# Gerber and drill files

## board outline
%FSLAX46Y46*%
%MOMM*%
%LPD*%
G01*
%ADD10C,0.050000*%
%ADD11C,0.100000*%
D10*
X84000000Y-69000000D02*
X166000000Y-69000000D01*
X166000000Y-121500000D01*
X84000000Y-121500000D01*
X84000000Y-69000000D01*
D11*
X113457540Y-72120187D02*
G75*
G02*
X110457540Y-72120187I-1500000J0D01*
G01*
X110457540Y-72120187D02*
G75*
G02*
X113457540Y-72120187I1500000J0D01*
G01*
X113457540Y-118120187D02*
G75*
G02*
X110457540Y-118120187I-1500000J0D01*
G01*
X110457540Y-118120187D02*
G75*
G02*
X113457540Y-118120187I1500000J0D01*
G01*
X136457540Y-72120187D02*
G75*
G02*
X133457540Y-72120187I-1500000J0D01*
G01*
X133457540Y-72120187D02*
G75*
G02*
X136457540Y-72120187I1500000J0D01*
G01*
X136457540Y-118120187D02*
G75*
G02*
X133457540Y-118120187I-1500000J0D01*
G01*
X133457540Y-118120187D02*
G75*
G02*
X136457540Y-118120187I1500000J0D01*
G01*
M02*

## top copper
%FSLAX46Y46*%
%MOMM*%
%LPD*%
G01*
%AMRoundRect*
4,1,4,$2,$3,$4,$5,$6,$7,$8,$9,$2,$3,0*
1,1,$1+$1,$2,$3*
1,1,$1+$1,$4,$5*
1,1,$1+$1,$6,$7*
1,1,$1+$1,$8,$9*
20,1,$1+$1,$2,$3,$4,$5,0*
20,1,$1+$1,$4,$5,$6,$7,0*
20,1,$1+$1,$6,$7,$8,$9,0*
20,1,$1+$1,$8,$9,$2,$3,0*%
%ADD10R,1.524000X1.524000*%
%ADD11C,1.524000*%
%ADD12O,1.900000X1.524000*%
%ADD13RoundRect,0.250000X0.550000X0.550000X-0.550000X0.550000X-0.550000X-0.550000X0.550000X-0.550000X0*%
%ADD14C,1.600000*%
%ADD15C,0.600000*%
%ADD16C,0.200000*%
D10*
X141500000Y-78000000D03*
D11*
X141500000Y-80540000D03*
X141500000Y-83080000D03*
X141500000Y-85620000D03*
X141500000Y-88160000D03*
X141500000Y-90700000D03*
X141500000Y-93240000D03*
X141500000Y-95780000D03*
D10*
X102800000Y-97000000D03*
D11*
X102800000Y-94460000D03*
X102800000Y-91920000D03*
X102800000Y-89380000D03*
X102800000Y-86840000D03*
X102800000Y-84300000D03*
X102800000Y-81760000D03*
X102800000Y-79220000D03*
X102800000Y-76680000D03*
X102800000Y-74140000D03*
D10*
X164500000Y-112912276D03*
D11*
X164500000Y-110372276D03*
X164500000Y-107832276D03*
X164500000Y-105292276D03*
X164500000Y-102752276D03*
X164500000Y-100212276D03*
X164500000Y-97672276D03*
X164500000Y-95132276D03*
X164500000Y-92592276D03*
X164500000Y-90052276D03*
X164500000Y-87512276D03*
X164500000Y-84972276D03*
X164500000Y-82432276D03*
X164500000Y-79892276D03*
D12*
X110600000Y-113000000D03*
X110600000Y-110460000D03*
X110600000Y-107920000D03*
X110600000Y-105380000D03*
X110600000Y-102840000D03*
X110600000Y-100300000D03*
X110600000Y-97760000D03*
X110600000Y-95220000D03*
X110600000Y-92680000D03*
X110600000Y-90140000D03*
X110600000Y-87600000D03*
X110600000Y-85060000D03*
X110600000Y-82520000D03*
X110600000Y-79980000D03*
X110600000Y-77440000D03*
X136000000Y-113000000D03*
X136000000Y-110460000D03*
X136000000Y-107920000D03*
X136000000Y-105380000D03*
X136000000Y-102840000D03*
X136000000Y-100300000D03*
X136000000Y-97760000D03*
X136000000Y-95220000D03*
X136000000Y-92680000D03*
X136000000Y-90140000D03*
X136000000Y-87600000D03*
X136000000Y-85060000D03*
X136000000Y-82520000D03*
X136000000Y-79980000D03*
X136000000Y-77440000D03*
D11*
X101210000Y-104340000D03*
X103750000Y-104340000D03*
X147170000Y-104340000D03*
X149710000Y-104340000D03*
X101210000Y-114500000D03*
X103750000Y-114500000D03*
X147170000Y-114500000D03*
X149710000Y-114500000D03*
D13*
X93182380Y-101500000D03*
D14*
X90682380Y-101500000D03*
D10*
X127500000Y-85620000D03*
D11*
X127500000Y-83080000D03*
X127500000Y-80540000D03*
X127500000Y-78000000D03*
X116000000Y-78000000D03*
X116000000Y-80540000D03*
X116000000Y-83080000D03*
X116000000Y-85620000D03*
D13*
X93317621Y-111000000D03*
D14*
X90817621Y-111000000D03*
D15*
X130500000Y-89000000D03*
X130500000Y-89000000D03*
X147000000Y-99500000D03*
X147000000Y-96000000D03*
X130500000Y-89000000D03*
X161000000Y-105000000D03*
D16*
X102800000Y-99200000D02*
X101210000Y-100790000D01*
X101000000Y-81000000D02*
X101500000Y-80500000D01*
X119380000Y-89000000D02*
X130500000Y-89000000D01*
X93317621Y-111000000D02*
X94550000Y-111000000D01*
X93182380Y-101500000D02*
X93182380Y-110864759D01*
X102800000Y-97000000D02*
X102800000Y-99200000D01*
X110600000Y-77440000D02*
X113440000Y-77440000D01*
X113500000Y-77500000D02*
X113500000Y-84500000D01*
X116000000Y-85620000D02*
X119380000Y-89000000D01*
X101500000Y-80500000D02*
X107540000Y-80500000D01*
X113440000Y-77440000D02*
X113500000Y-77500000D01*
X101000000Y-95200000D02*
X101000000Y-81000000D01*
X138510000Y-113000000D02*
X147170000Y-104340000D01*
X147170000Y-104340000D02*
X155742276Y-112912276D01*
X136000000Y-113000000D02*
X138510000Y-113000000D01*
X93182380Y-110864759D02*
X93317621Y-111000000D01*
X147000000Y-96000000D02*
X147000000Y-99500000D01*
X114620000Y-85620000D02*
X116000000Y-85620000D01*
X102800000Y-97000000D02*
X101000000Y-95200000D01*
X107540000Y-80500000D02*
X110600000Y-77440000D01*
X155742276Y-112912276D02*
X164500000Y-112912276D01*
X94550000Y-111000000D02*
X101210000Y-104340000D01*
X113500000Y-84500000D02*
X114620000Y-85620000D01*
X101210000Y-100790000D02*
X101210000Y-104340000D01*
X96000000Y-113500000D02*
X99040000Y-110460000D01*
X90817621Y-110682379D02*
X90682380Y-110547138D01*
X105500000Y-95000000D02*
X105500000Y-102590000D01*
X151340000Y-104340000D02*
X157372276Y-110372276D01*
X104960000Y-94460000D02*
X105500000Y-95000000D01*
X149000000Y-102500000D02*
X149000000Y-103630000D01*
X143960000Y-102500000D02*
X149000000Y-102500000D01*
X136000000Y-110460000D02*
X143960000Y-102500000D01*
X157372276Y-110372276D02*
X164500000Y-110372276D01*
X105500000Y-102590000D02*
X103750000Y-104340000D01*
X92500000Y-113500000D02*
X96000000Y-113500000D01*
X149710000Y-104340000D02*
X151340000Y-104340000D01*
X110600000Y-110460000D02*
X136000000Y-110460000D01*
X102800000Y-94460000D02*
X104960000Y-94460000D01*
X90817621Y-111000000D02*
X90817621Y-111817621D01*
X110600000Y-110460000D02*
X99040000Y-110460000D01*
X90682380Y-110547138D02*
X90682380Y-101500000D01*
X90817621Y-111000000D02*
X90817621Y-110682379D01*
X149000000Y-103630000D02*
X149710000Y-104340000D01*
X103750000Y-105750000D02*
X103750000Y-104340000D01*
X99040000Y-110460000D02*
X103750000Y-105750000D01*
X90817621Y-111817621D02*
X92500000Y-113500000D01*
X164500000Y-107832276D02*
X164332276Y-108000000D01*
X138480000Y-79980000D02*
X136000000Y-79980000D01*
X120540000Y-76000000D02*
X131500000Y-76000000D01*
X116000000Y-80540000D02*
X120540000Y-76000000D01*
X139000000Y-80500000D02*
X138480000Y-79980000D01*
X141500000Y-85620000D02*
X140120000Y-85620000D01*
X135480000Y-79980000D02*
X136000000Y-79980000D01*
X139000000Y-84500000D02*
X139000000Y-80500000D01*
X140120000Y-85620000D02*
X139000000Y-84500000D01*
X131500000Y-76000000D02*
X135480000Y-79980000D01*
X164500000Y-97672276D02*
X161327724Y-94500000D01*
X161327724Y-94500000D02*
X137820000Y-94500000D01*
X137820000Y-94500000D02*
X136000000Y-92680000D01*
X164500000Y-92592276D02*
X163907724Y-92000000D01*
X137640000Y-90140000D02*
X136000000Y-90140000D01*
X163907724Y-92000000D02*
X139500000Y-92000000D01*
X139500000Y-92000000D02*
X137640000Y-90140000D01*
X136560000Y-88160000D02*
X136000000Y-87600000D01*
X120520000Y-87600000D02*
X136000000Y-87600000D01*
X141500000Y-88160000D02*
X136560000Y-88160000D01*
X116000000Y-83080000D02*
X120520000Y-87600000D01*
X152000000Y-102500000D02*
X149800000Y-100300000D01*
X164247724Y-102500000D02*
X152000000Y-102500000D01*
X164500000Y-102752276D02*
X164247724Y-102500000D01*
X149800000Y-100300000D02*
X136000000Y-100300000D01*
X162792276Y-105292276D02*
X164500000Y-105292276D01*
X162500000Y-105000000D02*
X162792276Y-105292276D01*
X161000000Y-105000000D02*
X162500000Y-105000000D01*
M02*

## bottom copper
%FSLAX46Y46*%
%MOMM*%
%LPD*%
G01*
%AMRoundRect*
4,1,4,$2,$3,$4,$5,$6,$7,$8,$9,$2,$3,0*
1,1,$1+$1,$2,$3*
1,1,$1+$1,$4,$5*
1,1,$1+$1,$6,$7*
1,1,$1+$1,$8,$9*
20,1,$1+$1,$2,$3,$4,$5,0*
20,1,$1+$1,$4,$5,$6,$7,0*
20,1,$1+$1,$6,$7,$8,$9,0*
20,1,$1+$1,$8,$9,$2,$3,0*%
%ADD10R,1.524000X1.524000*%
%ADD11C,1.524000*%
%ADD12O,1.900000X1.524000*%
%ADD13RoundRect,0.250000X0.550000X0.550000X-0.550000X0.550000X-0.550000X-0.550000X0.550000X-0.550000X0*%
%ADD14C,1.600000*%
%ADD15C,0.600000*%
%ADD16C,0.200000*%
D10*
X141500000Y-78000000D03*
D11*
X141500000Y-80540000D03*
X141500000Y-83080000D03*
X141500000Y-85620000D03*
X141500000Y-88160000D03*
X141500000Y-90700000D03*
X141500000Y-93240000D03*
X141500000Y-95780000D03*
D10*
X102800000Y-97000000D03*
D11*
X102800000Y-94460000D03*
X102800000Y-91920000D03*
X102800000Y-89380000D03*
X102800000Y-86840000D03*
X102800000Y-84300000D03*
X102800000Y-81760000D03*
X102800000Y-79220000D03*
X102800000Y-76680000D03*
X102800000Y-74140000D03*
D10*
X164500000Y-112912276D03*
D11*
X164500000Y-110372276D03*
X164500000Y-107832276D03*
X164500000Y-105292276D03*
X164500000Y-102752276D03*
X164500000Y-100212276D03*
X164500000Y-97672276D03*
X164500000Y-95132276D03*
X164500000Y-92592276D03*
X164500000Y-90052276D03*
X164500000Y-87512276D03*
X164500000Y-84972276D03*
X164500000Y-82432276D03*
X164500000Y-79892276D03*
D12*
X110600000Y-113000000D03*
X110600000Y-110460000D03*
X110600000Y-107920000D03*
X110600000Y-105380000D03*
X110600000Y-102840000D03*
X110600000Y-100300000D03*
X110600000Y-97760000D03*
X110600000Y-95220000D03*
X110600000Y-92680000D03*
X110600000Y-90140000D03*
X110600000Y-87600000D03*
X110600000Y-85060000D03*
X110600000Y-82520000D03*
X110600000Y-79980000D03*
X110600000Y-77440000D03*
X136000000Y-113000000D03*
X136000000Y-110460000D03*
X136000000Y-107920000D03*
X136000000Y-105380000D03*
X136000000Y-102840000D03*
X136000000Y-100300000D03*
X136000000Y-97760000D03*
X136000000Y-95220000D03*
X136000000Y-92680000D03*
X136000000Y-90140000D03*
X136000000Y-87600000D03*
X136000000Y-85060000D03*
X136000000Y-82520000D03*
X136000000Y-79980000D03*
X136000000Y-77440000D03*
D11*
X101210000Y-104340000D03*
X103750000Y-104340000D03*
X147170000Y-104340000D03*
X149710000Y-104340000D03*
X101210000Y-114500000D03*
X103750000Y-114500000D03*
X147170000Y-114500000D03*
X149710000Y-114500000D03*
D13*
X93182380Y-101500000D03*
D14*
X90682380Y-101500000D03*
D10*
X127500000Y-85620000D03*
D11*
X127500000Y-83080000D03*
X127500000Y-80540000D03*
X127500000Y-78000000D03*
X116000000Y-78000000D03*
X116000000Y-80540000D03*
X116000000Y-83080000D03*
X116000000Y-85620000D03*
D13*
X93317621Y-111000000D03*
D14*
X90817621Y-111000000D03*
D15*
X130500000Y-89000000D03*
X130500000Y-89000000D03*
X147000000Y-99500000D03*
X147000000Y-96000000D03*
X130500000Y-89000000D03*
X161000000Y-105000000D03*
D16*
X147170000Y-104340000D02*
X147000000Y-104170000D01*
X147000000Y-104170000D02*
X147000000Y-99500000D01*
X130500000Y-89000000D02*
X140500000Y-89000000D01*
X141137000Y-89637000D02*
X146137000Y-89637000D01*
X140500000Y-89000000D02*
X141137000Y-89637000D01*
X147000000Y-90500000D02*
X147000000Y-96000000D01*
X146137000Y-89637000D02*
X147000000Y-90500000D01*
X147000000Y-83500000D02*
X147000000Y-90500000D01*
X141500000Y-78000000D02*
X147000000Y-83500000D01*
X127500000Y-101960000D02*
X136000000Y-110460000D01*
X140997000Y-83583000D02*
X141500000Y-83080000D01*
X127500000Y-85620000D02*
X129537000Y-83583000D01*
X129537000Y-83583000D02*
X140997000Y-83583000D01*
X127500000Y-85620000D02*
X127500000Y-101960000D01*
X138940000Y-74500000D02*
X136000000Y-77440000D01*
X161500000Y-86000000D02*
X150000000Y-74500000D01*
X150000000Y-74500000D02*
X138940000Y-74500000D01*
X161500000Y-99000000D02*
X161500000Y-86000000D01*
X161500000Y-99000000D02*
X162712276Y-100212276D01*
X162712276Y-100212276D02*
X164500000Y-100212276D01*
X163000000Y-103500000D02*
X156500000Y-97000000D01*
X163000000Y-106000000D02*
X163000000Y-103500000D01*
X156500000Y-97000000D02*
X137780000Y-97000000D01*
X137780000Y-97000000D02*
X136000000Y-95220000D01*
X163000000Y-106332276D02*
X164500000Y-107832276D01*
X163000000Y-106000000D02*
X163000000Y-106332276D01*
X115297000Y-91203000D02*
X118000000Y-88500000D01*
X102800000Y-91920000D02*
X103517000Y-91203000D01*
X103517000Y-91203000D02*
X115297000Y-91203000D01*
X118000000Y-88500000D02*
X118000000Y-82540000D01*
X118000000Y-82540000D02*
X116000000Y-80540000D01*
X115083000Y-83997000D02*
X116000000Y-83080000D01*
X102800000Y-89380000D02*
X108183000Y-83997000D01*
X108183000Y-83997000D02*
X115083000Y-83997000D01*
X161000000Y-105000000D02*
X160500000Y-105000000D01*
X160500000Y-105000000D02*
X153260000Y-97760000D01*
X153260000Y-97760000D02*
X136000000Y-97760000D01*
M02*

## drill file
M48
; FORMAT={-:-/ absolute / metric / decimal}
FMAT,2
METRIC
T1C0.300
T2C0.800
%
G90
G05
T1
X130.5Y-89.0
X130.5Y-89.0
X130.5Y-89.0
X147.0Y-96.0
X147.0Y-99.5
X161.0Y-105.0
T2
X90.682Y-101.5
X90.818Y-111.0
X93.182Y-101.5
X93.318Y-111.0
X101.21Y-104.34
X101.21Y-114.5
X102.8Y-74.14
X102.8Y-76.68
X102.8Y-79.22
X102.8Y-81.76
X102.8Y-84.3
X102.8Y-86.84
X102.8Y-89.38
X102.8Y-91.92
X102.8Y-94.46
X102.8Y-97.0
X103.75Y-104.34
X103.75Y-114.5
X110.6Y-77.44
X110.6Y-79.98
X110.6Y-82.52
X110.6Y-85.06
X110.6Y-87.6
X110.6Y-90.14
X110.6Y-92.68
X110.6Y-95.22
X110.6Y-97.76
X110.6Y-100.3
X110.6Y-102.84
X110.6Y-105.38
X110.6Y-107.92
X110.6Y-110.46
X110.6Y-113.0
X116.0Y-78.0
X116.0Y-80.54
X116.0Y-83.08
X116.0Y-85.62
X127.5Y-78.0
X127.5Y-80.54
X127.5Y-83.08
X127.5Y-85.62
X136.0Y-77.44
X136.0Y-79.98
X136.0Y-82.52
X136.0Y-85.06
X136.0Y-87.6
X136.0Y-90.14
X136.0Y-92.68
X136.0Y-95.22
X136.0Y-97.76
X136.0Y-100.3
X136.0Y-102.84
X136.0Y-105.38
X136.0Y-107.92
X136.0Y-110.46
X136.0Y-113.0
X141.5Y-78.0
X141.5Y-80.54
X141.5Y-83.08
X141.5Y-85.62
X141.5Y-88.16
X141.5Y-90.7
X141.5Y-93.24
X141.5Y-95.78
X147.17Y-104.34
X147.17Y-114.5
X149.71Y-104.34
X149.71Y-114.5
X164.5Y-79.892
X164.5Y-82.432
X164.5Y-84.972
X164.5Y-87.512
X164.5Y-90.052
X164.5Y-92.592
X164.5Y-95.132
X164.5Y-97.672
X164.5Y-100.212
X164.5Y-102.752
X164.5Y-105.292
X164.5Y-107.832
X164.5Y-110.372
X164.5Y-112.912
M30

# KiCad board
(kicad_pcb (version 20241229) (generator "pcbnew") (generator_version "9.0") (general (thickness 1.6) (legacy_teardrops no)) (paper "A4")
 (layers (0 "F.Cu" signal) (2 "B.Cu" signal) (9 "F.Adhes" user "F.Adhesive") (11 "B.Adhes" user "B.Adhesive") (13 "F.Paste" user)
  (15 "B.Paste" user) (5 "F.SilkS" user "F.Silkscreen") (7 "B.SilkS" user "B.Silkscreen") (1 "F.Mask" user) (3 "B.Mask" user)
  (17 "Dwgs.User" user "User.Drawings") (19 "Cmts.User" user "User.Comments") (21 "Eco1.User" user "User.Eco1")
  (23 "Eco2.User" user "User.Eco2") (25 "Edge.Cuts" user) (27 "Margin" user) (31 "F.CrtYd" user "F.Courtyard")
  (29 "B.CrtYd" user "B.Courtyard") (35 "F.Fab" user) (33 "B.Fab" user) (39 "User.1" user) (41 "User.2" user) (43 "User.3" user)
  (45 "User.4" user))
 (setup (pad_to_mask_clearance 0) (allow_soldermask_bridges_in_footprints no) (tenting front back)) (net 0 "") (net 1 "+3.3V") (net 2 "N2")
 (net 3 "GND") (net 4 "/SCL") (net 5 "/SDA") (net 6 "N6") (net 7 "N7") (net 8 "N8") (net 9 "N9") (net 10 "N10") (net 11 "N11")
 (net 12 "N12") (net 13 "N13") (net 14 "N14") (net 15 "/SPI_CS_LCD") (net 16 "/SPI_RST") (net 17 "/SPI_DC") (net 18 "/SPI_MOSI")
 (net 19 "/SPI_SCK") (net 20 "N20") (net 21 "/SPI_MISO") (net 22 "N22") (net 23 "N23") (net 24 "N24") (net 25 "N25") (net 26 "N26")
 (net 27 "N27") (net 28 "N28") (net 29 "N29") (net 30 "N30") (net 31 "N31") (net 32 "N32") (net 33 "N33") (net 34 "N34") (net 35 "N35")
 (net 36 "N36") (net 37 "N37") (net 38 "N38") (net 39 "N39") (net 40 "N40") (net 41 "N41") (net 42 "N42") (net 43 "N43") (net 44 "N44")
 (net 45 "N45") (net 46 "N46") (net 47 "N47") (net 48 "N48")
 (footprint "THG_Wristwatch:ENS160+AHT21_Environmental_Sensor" (layer "F.Cu") (at 149.6 86.92 -90)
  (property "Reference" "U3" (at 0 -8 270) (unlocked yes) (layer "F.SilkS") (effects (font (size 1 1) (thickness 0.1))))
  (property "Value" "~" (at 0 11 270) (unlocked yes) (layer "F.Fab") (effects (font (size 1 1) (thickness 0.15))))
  (pad "1" thru_hole rect (at -8.92 8.1 270) (size 1.524 1.524) (drill 0.8) (layers "*.Cu" "*.Mask") (remove_unused_layers no)
   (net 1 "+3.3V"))
  (pad "2" thru_hole circle (at -6.38 8.1 270) (size 1.524 1.524) (drill 0.8) (layers "*.Cu" "*.Mask") (remove_unused_layers no)
   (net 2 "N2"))
  (pad "3" thru_hole circle (at -3.84 8.1 270) (size 1.524 1.524) (drill 0.8) (layers "*.Cu" "*.Mask") (remove_unused_layers no)
   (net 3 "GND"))
  (pad "4" thru_hole circle (at -1.3 8.1 270) (size 1.524 1.524) (drill 0.8) (layers "*.Cu" "*.Mask") (remove_unused_layers no)
   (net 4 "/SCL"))
  (pad "5" thru_hole circle (at 1.24 8.1 270) (size 1.524 1.524) (drill 0.8) (layers "*.Cu" "*.Mask") (remove_unused_layers no)
   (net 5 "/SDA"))
  (pad "6" thru_hole circle (at 3.78 8.1 270) (size 1.524 1.524) (drill 0.8) (layers "*.Cu" "*.Mask") (remove_unused_layers no) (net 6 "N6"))
  (pad "7" thru_hole circle (at 6.32 8.1 270) (size 1.524 1.524) (drill 0.8) (layers "*.Cu" "*.Mask") (remove_unused_layers no) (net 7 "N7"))
  (pad "8" thru_hole circle (at 8.86 8.1 270) (size 1.524 1.524) (drill 0.8) (layers "*.Cu" "*.Mask") (remove_unused_layers no) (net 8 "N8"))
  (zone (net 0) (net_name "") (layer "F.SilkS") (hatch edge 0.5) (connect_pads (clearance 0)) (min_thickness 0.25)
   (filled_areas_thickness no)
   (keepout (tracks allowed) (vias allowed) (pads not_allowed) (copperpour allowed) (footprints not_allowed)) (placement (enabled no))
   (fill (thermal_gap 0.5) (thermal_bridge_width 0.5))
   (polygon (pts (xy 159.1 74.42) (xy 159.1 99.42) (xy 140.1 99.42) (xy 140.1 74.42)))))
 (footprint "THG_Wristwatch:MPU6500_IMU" (layer "F.Cu") (at 96 85.5 180)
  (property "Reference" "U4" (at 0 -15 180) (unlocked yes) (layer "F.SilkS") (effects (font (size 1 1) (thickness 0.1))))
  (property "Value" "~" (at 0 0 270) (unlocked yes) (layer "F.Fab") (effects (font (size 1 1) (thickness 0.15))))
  (pad "1" thru_hole rect (at -6.8 -11.5 180) (size 1.524 1.524) (drill 0.8) (layers "*.Cu" "*.Mask") (remove_unused_layers no)
   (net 1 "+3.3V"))
  (pad "2" thru_hole circle (at -6.8 -8.96 180) (size 1.524 1.524) (drill 0.8) (layers "*.Cu" "*.Mask") (remove_unused_layers no)
   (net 3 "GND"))
  (pad "3" thru_hole circle (at -6.8 -6.42 180) (size 1.524 1.524) (drill 0.8) (layers "*.Cu" "*.Mask") (remove_unused_layers no)
   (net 4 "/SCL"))
  (pad "4" thru_hole circle (at -6.8 -3.88 180) (size 1.524 1.524) (drill 0.8) (layers "*.Cu" "*.Mask") (remove_unused_layers no)
   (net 5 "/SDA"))
  (pad "5" thru_hole circle (at -6.8 -1.34 180) (size 1.524 1.524) (drill 0.8) (layers "*.Cu" "*.Mask") (remove_unused_layers no)
   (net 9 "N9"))
  (pad "6" thru_hole circle (at -6.8 1.2 180) (size 1.524 1.524) (drill 0.8) (layers "*.Cu" "*.Mask") (remove_unused_layers no)
   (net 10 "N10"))
  (pad "7" thru_hole circle (at -6.8 3.74 180) (size 1.524 1.524) (drill 0.8) (layers "*.Cu" "*.Mask") (remove_unused_layers no)
   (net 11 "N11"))
  (pad "8" thru_hole circle (at -6.8 6.28 180) (size 1.524 1.524) (drill 0.8) (layers "*.Cu" "*.Mask") (remove_unused_layers no)
   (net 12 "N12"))
  (pad "9" thru_hole circle (at -6.8 8.82 180) (size 1.524 1.524) (drill 0.8) (layers "*.Cu" "*.Mask") (remove_unused_layers no)
   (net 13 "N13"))
  (pad "10" thru_hole circle (at -6.8 11.36 180) (size 1.524 1.524) (drill 0.8) (layers "*.Cu" "*.Mask") (remove_unused_layers no)
   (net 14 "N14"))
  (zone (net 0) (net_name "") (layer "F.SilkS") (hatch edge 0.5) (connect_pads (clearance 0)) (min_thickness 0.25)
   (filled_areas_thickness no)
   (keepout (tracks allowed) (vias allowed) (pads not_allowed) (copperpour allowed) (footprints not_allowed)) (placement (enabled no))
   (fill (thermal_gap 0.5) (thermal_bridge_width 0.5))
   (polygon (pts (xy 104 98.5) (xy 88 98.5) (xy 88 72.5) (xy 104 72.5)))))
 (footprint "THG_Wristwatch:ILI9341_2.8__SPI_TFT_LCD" (layer "F.Cu") (at 125 96.372276)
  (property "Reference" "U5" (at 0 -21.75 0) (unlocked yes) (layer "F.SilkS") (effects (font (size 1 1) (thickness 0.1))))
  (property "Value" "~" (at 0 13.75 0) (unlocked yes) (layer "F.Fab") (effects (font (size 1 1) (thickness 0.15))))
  (pad "1" thru_hole rect (at 39.5 16.54) (size 1.524 1.524) (drill 0.8) (layers "*.Cu" "*.Mask") (remove_unused_layers no) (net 1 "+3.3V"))
  (pad "2" thru_hole circle (at 39.5 14) (size 1.524 1.524) (drill 0.8) (layers "*.Cu" "*.Mask") (remove_unused_layers no) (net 3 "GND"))
  (pad "3" thru_hole circle (at 39.5 11.46) (size 1.524 1.524) (drill 0.8) (layers "*.Cu" "*.Mask") (remove_unused_layers no)
   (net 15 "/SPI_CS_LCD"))
  (pad "4" thru_hole circle (at 39.5 8.92) (size 1.524 1.524) (drill 0.8) (layers "*.Cu" "*.Mask") (remove_unused_layers no)
   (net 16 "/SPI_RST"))
  (pad "5" thru_hole circle (at 39.5 6.38) (size 1.524 1.524) (drill 0.8) (layers "*.Cu" "*.Mask") (remove_unused_layers no)
   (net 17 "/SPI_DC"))
  (pad "6" thru_hole circle (at 39.5 3.84) (size 1.524 1.524) (drill 0.8) (layers "*.Cu" "*.Mask") (remove_unused_layers no)
   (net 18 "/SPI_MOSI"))
  (pad "7" thru_hole circle (at 39.5 1.3) (size 1.524 1.524) (drill 0.8) (layers "*.Cu" "*.Mask") (remove_unused_layers no)
   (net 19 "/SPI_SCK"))
  (pad "8" thru_hole circle (at 39.5 -1.24) (size 1.524 1.524) (drill 0.8) (layers "*.Cu" "*.Mask") (remove_unused_layers no) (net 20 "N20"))
  (pad "9" thru_hole circle (at 39.5 -3.78) (size 1.524 1.524) (drill 0.8) (layers "*.Cu" "*.Mask") (remove_unused_layers no)
   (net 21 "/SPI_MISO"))
  (pad "10" thru_hole circle (at 39.5 -6.32) (size 1.524 1.524) (drill 0.8) (layers "*.Cu" "*.Mask") (remove_unused_layers no)
   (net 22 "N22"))
  (pad "11" thru_hole circle (at 39.5 -8.86) (size 1.524 1.524) (drill 0.8) (layers "*.Cu" "*.Mask") (remove_unused_layers no)
   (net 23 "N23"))
  (pad "12" thru_hole circle (at 39.5 -11.4) (size 1.524 1.524) (drill 0.8) (layers "*.Cu" "*.Mask") (remove_unused_layers no)
   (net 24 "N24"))
  (pad "13" thru_hole circle (at 39.5 -13.94) (size 1.524 1.524) (drill 0.8) (layers "*.Cu" "*.Mask") (remove_unused_layers no)
   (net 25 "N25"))
  (pad "14" thru_hole circle (at 39.5 -16.48) (size 1.524 1.524) (drill 0.8) (layers "*.Cu" "*.Mask") (remove_unused_layers no)
   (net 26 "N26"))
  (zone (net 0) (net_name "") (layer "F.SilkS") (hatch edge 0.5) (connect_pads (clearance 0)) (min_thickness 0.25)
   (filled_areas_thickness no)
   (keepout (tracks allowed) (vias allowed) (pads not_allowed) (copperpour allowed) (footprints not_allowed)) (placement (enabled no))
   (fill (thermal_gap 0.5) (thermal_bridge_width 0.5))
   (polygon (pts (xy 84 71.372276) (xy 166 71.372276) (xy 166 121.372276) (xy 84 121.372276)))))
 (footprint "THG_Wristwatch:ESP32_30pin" (layer "F.Cu") (at 122.52754 95.980187)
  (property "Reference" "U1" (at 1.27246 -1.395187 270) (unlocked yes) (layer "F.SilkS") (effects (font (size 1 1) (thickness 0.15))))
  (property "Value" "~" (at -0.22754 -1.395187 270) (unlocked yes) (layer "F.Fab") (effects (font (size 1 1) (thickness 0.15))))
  (fp_circle (center -10.57 -23.86) (end -10.57 -22.36) (stroke (width 0.1) (type default)) (fill no) (layer "Edge.Cuts"))
  (fp_circle (center -10.57 22.14) (end -10.57 23.64) (stroke (width 0.1) (type default)) (fill no) (layer "Edge.Cuts"))
  (fp_circle (center 12.43 -23.86) (end 12.43 -22.36) (stroke (width 0.1) (type default)) (fill no) (layer "Edge.Cuts"))
  (fp_circle (center 12.43 22.14) (end 12.43 23.64) (stroke (width 0.1) (type default)) (fill no) (layer "Edge.Cuts"))
  (pad "1" thru_hole oval (at -11.92754 17.019813 270) (size 1.524 1.9) (drill 0.8) (layers "*.Cu" "*.Mask") (remove_unused_layers no)
   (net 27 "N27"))
  (pad "2" thru_hole oval (at -11.92754 14.479813 270) (size 1.524 1.9) (drill 0.8) (layers "*.Cu" "*.Mask") (remove_unused_layers no)
   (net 3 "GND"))
  (pad "3" thru_hole oval (at -11.92754 11.939813 270) (size 1.524 1.9) (drill 0.8) (layers "*.Cu" "*.Mask") (remove_unused_layers no)
   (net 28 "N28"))
  (pad "4" thru_hole oval (at -11.92754 9.399813 270) (size 1.524 1.9) (drill 0.8) (layers "*.Cu" "*.Mask") (remove_unused_layers no)
   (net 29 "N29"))
  (pad "5" thru_hole oval (at -11.92754 6.859813 270) (size 1.524 1.9) (drill 0.8) (layers "*.Cu" "*.Mask") (remove_unused_layers no)
   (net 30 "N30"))
  (pad "6" thru_hole oval (at -11.92754 4.319813 270) (size 1.524 1.9) (drill 0.8) (layers "*.Cu" "*.Mask") (remove_unused_layers no)
   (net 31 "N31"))
  (pad "7" thru_hole oval (at -11.92754 1.779813 270) (size 1.524 1.9) (drill 0.8) (layers "*.Cu" "*.Mask") (remove_unused_layers no)
   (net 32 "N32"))
  (pad "8" thru_hole oval (at -11.92754 -0.760187 270) (size 1.524 1.9) (drill 0.8) (layers "*.Cu" "*.Mask") (remove_unused_layers no)
   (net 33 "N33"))
  (pad "9" thru_hole oval (at -11.92754 -3.300187 270) (size 1.524 1.9) (drill 0.8) (layers "*.Cu" "*.Mask") (remove_unused_layers no)
   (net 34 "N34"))
  (pad "10" thru_hole oval (at -11.92754 -5.840187 270) (size 1.524 1.9) (drill 0.8) (layers "*.Cu" "*.Mask") (remove_unused_layers no)
   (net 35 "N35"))
  (pad "11" thru_hole oval (at -11.92754 -8.380187 270) (size 1.524 1.9) (drill 0.8) (layers "*.Cu" "*.Mask") (remove_unused_layers no)
   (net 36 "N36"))
  (pad "12" thru_hole oval (at -11.92754 -10.920187 270) (size 1.524 1.9) (drill 0.8) (layers "*.Cu" "*.Mask") (remove_unused_layers no)
   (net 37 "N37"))
  (pad "13" thru_hole oval (at -11.92754 -13.460187 270) (size 1.524 1.9) (drill 0.8) (layers "*.Cu" "*.Mask") (remove_unused_layers no)
   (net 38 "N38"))
  (pad "14" thru_hole oval (at -11.92754 -16.000187 270) (size 1.524 1.9) (drill 0.8) (layers "*.Cu" "*.Mask") (remove_unused_layers no)
   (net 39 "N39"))
  (pad "15" thru_hole oval (at -11.92754 -18.540187 270) (size 1.524 1.9) (drill 0.8) (layers "*.Cu" "*.Mask") (remove_unused_layers no)
   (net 1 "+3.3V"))
  (pad "16" thru_hole oval (at 13.47246 17.019813 270) (size 1.524 1.9) (drill 0.8) (layers "*.Cu" "*.Mask") (remove_unused_layers no)
   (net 1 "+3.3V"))
  (pad "17" thru_hole oval (at 13.47246 14.479813 270) (size 1.524 1.9) (drill 0.8) (layers "*.Cu" "*.Mask") (remove_unused_layers no)
   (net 3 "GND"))
  (pad "18" thru_hole oval (at 13.47246 11.939813 270) (size 1.524 1.9) (drill 0.8) (layers "*.Cu" "*.Mask") (remove_unused_layers no)
   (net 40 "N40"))
  (pad "19" thru_hole oval (at 13.47246 9.399813 270) (size 1.524 1.9) (drill 0.8) (layers "*.Cu" "*.Mask") (remove_unused_layers no)
   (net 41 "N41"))
  (pad "20" thru_hole oval (at 13.47246 6.859813 270) (size 1.524 1.9) (drill 0.8) (layers "*.Cu" "*.Mask" "Dwgs.User")
   (remove_unused_layers no) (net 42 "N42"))
  (pad "21" thru_hole oval (at 13.47246 4.319813 270) (size 1.524 1.9) (drill 0.8) (layers "*.Cu" "*.Mask") (remove_unused_layers no)
   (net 17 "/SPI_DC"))
  (pad "22" thru_hole oval (at 13.47246 1.779813 270) (size 1.524 1.9) (drill 0.8) (layers "*.Cu" "*.Mask") (remove_unused_layers no)
   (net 16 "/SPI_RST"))
  (pad "23" thru_hole oval (at 13.47246 -0.760187 270) (size 1.524 1.9) (drill 0.8) (layers "*.Cu" "*.Mask") (remove_unused_layers no)
   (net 15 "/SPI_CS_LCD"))
  (pad "24" thru_hole oval (at 13.47246 -3.300187 270) (size 1.524 1.9) (drill 0.8) (layers "*.Cu" "*.Mask") (remove_unused_layers no)
   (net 19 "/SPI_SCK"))
  (pad "25" thru_hole oval (at 13.47246 -5.840187 270) (size 1.524 1.9) (drill 0.8) (layers "*.Cu" "*.Mask") (remove_unused_layers no)
   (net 21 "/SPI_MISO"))
  (pad "26" thru_hole oval (at 13.47246 -8.380187 270) (size 1.524 1.9) (drill 0.8) (layers "*.Cu" "*.Mask") (remove_unused_layers no)
   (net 5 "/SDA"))
  (pad "27" thru_hole oval (at 13.47246 -10.920187 270) (size 1.524 1.9) (drill 0.8) (layers "*.Cu" "*.Mask") (remove_unused_layers no)
   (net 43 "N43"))
  (pad "28" thru_hole oval (at 13.47246 -13.460187 270) (size 1.524 1.9) (drill 0.8) (layers "*.Cu" "*.Mask") (remove_unused_layers no)
   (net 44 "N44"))
  (pad "29" thru_hole oval (at 13.47246 -16.000187 270) (size 1.524 1.9) (drill 0.8) (layers "*.Cu" "*.Mask") (remove_unused_layers no)
   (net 4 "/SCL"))
  (pad "30" thru_hole oval (at 13.47246 -18.540187 270) (size 1.524 1.9) (drill 0.8) (layers "*.Cu" "*.Mask") (remove_unused_layers no)
   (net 18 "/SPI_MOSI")))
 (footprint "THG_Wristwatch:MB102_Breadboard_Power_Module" (layer "B.Cu") (at 125.5 112)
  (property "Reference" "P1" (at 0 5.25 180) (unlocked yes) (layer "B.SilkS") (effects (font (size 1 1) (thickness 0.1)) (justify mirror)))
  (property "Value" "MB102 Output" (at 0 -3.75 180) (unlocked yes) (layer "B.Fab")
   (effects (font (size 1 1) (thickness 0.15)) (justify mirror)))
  (pad "1" thru_hole circle (at -24.29 -7.66) (size 1.524 1.524) (drill 0.8) (layers "*.Cu" "*.Mask") (remove_unused_layers no)
   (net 1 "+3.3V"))
  (pad "2" thru_hole circle (at -21.75 -7.66) (size 1.524 1.524) (drill 0.8) (layers "*.Cu" "*.Mask") (remove_unused_layers no)
   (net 3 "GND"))
  (pad "3" thru_hole circle (at 21.67 -7.66) (size 1.524 1.524) (drill 0.8) (layers "*.Cu" "*.Mask") (remove_unused_layers no)
   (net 1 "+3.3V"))
  (pad "4" thru_hole circle (at 24.21 -7.66) (size 1.524 1.524) (drill 0.8) (layers "*.Cu" "*.Mask") (remove_unused_layers no) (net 3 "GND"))
  (pad "5" thru_hole circle (at -24.29 2.5) (size 1.524 1.524) (drill 0.8) (layers "*.Cu" "*.Mask") (remove_unused_layers no))
  (pad "6" thru_hole circle (at -21.75 2.5) (size 1.524 1.524) (drill 0.8) (layers "*.Cu" "*.Mask") (remove_unused_layers no))
  (pad "7" thru_hole circle (at 21.67 2.5) (size 1.524 1.524) (drill 0.8) (layers "*.Cu" "*.Mask") (remove_unused_layers no))
  (pad "8" thru_hole circle (at 24.21 2.5) (size 1.524 1.524) (drill 0.8) (layers "*.Cu" "*.Mask") (remove_unused_layers no))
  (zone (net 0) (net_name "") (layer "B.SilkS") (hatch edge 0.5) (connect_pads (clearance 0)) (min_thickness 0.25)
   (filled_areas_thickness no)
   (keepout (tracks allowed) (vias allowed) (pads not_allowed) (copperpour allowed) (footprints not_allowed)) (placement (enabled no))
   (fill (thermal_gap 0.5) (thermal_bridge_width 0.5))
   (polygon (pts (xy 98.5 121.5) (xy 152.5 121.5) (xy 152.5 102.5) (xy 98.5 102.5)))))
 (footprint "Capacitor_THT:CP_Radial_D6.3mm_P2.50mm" (layer "B.Cu") (at 93.18238 101.5 180)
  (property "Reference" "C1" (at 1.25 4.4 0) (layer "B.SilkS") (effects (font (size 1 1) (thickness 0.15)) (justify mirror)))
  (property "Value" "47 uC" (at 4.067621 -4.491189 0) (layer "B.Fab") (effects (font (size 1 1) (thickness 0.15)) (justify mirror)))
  (pad "1" thru_hole roundrect (at 0 0 180) (size 1.6 1.6) (drill 0.8) (layers "*.Cu" "*.Mask") (remove_unused_layers no)
   (roundrect_rratio 0.15625) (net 1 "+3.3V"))
  (pad "2" thru_hole circle (at 2.5 0 180) (size 1.6 1.6) (drill 0.8) (layers "*.Cu" "*.Mask") (remove_unused_layers no) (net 3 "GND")))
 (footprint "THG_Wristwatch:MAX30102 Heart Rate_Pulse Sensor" (layer "B.Cu") (at 121.8 81.7 180)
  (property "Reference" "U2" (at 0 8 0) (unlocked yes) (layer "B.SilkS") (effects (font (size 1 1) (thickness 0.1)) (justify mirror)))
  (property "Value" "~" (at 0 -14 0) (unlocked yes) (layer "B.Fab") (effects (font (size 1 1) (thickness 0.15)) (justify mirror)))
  (pad "1" thru_hole rect (at -5.7 -3.92 180) (size 1.524 1.524) (drill 0.8) (layers "*.Cu" "*.Mask") (remove_unused_layers no)
   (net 3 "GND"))
  (pad "2" thru_hole circle (at -5.7 -1.38 180) (size 1.524 1.524) (drill 0.8) (layers "*.Cu" "*.Mask") (remove_unused_layers no)
   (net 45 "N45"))
  (pad "3" thru_hole circle (at -5.7 1.16 180) (size 1.524 1.524) (drill 0.8) (layers "*.Cu" "*.Mask") (remove_unused_layers no)
   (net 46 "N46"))
  (pad "4" thru_hole circle (at -5.7 3.7 180) (size 1.524 1.524) (drill 0.8) (layers "*.Cu" "*.Mask") (remove_unused_layers no)
   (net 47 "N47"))
  (pad "5" thru_hole circle (at 5.8 3.7 180) (size 1.524 1.524) (drill 0.8) (layers "*.Cu" "*.Mask") (remove_unused_layers no)
   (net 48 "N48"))
  (pad "6" thru_hole circle (at 5.8 1.16 180) (size 1.524 1.524) (drill 0.8) (layers "*.Cu" "*.Mask") (remove_unused_layers no)
   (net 4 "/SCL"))
  (pad "7" thru_hole circle (at 5.8 -1.38 180) (size 1.524 1.524) (drill 0.8) (layers "*.Cu" "*.Mask") (remove_unused_layers no)
   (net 5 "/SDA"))
  (pad "8" thru_hole circle (at 5.8 -3.92 180) (size 1.524 1.524) (drill 0.8) (layers "*.Cu" "*.Mask") (remove_unused_layers no)
   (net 1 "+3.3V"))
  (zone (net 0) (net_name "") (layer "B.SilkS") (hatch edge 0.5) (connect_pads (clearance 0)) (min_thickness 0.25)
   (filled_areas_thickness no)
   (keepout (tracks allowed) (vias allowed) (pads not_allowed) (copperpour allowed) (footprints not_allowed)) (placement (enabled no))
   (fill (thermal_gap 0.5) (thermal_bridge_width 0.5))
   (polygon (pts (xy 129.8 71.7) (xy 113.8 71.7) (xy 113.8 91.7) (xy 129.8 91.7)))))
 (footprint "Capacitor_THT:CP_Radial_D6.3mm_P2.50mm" (layer "B.Cu") (at 93.317621 111 180)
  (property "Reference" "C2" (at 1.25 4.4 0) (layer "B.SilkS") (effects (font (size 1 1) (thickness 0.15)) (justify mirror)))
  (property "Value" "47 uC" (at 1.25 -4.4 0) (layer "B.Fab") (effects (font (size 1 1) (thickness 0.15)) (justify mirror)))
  (pad "1" thru_hole roundrect (at 0 0 180) (size 1.6 1.6) (drill 0.8) (layers "*.Cu" "*.Mask") (remove_unused_layers no)
   (roundrect_rratio 0.15625) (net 1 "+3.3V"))
  (pad "2" thru_hole circle (at 2.5 0 180) (size 1.6 1.6) (drill 0.8) (layers "*.Cu" "*.Mask") (remove_unused_layers no) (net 3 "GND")))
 (gr_rect (start 166 69) (end 84 121.5) (stroke (width 0.05) (type solid)) (fill no) (layer "Edge.Cuts"))
 (segment (start 102.8 99.2) (end 101.21 100.79) (width 0.2) (layer "F.Cu") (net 1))
 (segment (start 101 81) (end 101.5 80.5) (width 0.2) (layer "F.Cu") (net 1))
 (segment (start 119.38 89) (end 130.5 89) (width 0.2) (layer "F.Cu") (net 1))
 (segment (start 93.317621 111) (end 94.55 111) (width 0.2) (layer "F.Cu") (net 1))
 (segment (start 93.18238 101.5) (end 93.18238 110.864759) (width 0.2) (layer "F.Cu") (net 1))
 (segment (start 102.8 97) (end 102.8 99.2) (width 0.2) (layer "F.Cu") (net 1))
 (segment (start 110.6 77.44) (end 113.44 77.44) (width 0.2) (layer "F.Cu") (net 1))
 (segment (start 113.5 77.5) (end 113.5 84.5) (width 0.2) (layer "F.Cu") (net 1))
 (segment (start 116 85.62) (end 119.38 89) (width 0.2) (layer "F.Cu") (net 1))
 (segment (start 101.5 80.5) (end 107.54 80.5) (width 0.2) (layer "F.Cu") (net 1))
 (segment (start 113.44 77.44) (end 113.5 77.5) (width 0.2) (layer "F.Cu") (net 1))
 (segment (start 101 95.2) (end 101 81) (width 0.2) (layer "F.Cu") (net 1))
 (segment (start 138.51 113) (end 147.17 104.34) (width 0.2) (layer "F.Cu") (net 1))
 (segment (start 147.17 104.34) (end 155.742276 112.912276) (width 0.2) (layer "F.Cu") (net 1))
 (segment (start 136 113) (end 138.51 113) (width 0.2) (layer "F.Cu") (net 1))
 (segment (start 93.18238 110.864759) (end 93.317621 111) (width 0.2) (layer "F.Cu") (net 1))
 (segment (start 147 96) (end 147 99.5) (width 0.2) (layer "F.Cu") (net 1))
 (segment (start 114.62 85.62) (end 116 85.62) (width 0.2) (layer "F.Cu") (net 1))
 (segment (start 102.8 97) (end 101 95.2) (width 0.2) (layer "F.Cu") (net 1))
 (segment (start 107.54 80.5) (end 110.6 77.44) (width 0.2) (layer "F.Cu") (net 1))
 (segment (start 155.742276 112.912276) (end 164.5 112.912276) (width 0.2) (layer "F.Cu") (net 1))
 (segment (start 94.55 111) (end 101.21 104.34) (width 0.2) (layer "F.Cu") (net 1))
 (segment (start 113.5 84.5) (end 114.62 85.62) (width 0.2) (layer "F.Cu") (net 1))
 (segment (start 101.21 100.79) (end 101.21 104.34) (width 0.2) (layer "F.Cu") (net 1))
 (via (at 130.5 89) (size 0.6) (drill 0.3) (layers "F.Cu" "B.Cu") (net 1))
 (via (at 130.5 89) (size 0.6) (drill 0.3) (layers "F.Cu" "B.Cu") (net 1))
 (via (at 147 99.5) (size 0.6) (drill 0.3) (layers "F.Cu" "B.Cu") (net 1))
 (via (at 147 96) (size 0.6) (drill 0.3) (layers "F.Cu" "B.Cu") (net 1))
 (via (at 130.5 89) (size 0.6) (drill 0.3) (layers "F.Cu" "B.Cu") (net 1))
 (segment (start 147.17 104.34) (end 147 104.17) (width 0.2) (layer "B.Cu") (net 1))
 (segment (start 147 104.17) (end 147 99.5) (width 0.2) (layer "B.Cu") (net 1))
 (segment (start 130.5 89) (end 140.5 89) (width 0.2) (layer "B.Cu") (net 1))
 (segment (start 141.137 89.637) (end 146.137 89.637) (width 0.2) (layer "B.Cu") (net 1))
 (segment (start 140.5 89) (end 141.137 89.637) (width 0.2) (layer "B.Cu") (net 1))
 (segment (start 147 90.5) (end 147 96) (width 0.2) (layer "B.Cu") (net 1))
 (segment (start 146.137 89.637) (end 147 90.5) (width 0.2) (layer "B.Cu") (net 1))
 (segment (start 147 83.5) (end 147 90.5) (width 0.2) (layer "B.Cu") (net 1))
 (segment (start 141.5 78) (end 147 83.5) (width 0.2) (layer "B.Cu") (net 1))
 (segment (start 96 113.5) (end 99.04 110.46) (width 0.2) (layer "F.Cu") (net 3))
 (segment (start 90.817621 110.682379) (end 90.68238 110.547138) (width 0.2) (layer "F.Cu") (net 3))
 (segment (start 105.5 95) (end 105.5 102.59) (width 0.2) (layer "F.Cu") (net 3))
 (segment (start 151.34 104.34) (end 157.372276 110.372276) (width 0.2) (layer "F.Cu") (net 3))
 (segment (start 104.96 94.46) (end 105.5 95) (width 0.2) (layer "F.Cu") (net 3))
 (segment (start 149 102.5) (end 149 103.63) (width 0.2) (layer "F.Cu") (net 3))
 (segment (start 143.96 102.5) (end 149 102.5) (width 0.2) (layer "F.Cu") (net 3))
 (segment (start 136 110.46) (end 143.96 102.5) (width 0.2) (layer "F.Cu") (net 3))
 (segment (start 157.372276 110.372276) (end 164.5 110.372276) (width 0.2) (layer "F.Cu") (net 3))
 (segment (start 105.5 102.59) (end 103.75 104.34) (width 0.2) (layer "F.Cu") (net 3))
 (segment (start 92.5 113.5) (end 96 113.5) (width 0.2) (layer "F.Cu") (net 3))
 (segment (start 149.71 104.34) (end 151.34 104.34) (width 0.2) (layer "F.Cu") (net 3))
 (segment (start 110.6 110.46) (end 136 110.46) (width 0.2) (layer "F.Cu") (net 3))
 (segment (start 102.8 94.46) (end 104.96 94.46) (width 0.2) (layer "F.Cu") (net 3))
 (segment (start 90.817621 111) (end 90.817621 111.817621) (width 0.2) (layer "F.Cu") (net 3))
 (segment (start 110.6 110.46) (end 99.04 110.46) (width 0.2) (layer "F.Cu") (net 3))
 (segment (start 90.68238 110.547138) (end 90.68238 101.5) (width 0.2) (layer "F.Cu") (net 3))
 (segment (start 90.817621 111) (end 90.817621 110.682379) (width 0.2) (layer "F.Cu") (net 3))
 (segment (start 149 103.63) (end 149.71 104.34) (width 0.2) (layer "F.Cu") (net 3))
 (segment (start 103.75 105.75) (end 103.75 104.34) (width 0.2) (layer "F.Cu") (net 3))
 (segment (start 99.04 110.46) (end 103.75 105.75) (width 0.2) (layer "F.Cu") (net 3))
 (segment (start 90.817621 111.817621) (end 92.5 113.5) (width 0.2) (layer "F.Cu") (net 3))
 (segment (start 127.5 101.96) (end 136 110.46) (width 0.2) (layer "B.Cu") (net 3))
 (segment (start 140.997 83.583) (end 141.5 83.08) (width 0.2) (layer "B.Cu") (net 3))
 (segment (start 127.5 85.62) (end 129.537 83.583) (width 0.2) (layer "B.Cu") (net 3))
 (segment (start 129.537 83.583) (end 140.997 83.583) (width 0.2) (layer "B.Cu") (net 3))
 (segment (start 127.5 85.62) (end 127.5 101.96) (width 0.2) (layer "B.Cu") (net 3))
 (segment (start 138.94 74.5) (end 136 77.44) (width 0.2) (layer "B.Cu") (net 18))
 (segment (start 161.5 86) (end 150 74.5) (width 0.2) (layer "B.Cu") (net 18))
 (segment (start 150 74.5) (end 138.94 74.5) (width 0.2) (layer "B.Cu") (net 18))
 (segment (start 161.5 99) (end 161.5 86) (width 0.2) (layer "B.Cu") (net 18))
 (segment (start 161.5 99) (end 162.712276 100.212276) (width 0.2) (layer "B.Cu") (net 18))
 (segment (start 162.712276 100.212276) (end 164.5 100.212276) (width 0.2) (layer "B.Cu") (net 18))
 (segment (start 164.5 107.832276) (end 164.332276 108) (width 0.2) (layer "F.Cu") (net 15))
 (segment (start 163 103.5) (end 156.5 97) (width 0.2) (layer "B.Cu") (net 15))
 (segment (start 163 106) (end 163 103.5) (width 0.2) (layer "B.Cu") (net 15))
 (segment (start 156.5 97) (end 137.78 97) (width 0.2) (layer "B.Cu") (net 15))
 (segment (start 137.78 97) (end 136 95.22) (width 0.2) (layer "B.Cu") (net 15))
 (segment (start 163 106.332276) (end 164.5 107.832276) (width 0.2) (layer "B.Cu") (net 15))
 (segment (start 163 106) (end 163 106.332276) (width 0.2) (layer "B.Cu") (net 15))
 (segment (start 138.48 79.98) (end 136 79.98) (width 0.2) (layer "F.Cu") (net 4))
 (segment (start 120.54 76) (end 131.5 76) (width 0.2) (layer "F.Cu") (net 4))
 (segment (start 116 80.54) (end 120.54 76) (width 0.2) (layer "F.Cu") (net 4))
 (segment (start 139 80.5) (end 138.48 79.98) (width 0.2) (layer "F.Cu") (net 4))
 (segment (start 141.5 85.62) (end 140.12 85.62) (width 0.2) (layer "F.Cu") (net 4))
 (segment (start 135.48 79.98) (end 136 79.98) (width 0.2) (layer "F.Cu") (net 4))
 (segment (start 139 84.5) (end 139 80.5) (width 0.2) (layer "F.Cu") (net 4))
 (segment (start 140.12 85.62) (end 139 84.5) (width 0.2) (layer "F.Cu") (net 4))
 (segment (start 131.5 76) (end 135.48 79.98) (width 0.2) (layer "F.Cu") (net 4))
 (segment (start 115.297 91.203) (end 118 88.5) (width 0.2) (layer "B.Cu") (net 4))
 (segment (start 102.8 91.92) (end 103.517 91.203) (width 0.2) (layer "B.Cu") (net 4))
 (segment (start 103.517 91.203) (end 115.297 91.203) (width 0.2) (layer "B.Cu") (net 4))
 (segment (start 118 88.5) (end 118 82.54) (width 0.2) (layer "B.Cu") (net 4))
 (segment (start 118 82.54) (end 116 80.54) (width 0.2) (layer "B.Cu") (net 4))
 (segment (start 164.5 97.672276) (end 161.327724 94.5) (width 0.2) (layer "F.Cu") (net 19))
 (segment (start 161.327724 94.5) (end 137.82 94.5) (width 0.2) (layer "F.Cu") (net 19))
 (segment (start 137.82 94.5) (end 136 92.68) (width 0.2) (layer "F.Cu") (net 19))
 (segment (start 164.5 92.592276) (end 163.907724 92) (width 0.2) (layer "F.Cu") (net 21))
 (segment (start 137.64 90.14) (end 136 90.14) (width 0.2) (layer "F.Cu") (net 21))
 (segment (start 163.907724 92) (end 139.5 92) (width 0.2) (layer "F.Cu") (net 21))
 (segment (start 139.5 92) (end 137.64 90.14) (width 0.2) (layer "F.Cu") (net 21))
 (segment (start 136.56 88.16) (end 136 87.6) (width 0.2) (layer "F.Cu") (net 5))
 (segment (start 120.52 87.6) (end 136 87.6) (width 0.2) (layer "F.Cu") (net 5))
 (segment (start 141.5 88.16) (end 136.56 88.16) (width 0.2) (layer "F.Cu") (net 5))
 (segment (start 116 83.08) (end 120.52 87.6) (width 0.2) (layer "F.Cu") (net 5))
 (segment (start 115.083 83.997) (end 116 83.08) (width 0.2) (layer "B.Cu") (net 5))
 (segment (start 102.8 89.38) (end 108.183 83.997) (width 0.2) (layer "B.Cu") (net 5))
 (segment (start 108.183 83.997) (end 115.083 83.997) (width 0.2) (layer "B.Cu") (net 5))
 (segment (start 152 102.5) (end 149.8 100.3) (width 0.2) (layer "F.Cu") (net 17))
 (segment (start 164.247724 102.5) (end 152 102.5) (width 0.2) (layer "F.Cu") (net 17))
 (segment (start 164.5 102.752276) (end 164.247724 102.5) (width 0.2) (layer "F.Cu") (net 17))
 (segment (start 149.8 100.3) (end 136 100.3) (width 0.2) (layer "F.Cu") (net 17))
 (segment (start 162.792276 105.292276) (end 164.5 105.292276) (width 0.2) (layer "F.Cu") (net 16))
 (segment (start 162.5 105) (end 162.792276 105.292276) (width 0.2) (layer "F.Cu") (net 16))
 (segment (start 161 105) (end 162.5 105) (width 0.2) (layer "F.Cu") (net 16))
 (via (at 161 105) (size 0.6) (drill 0.3) (layers "F.Cu" "B.Cu") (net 16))
 (segment (start 161 105) (end 160.5 105) (width 0.2) (layer "B.Cu") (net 16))
 (segment (start 160.5 105) (end 153.26 97.76) (width 0.2) (layer "B.Cu") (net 16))
 (segment (start 153.26 97.76) (end 136 97.76) (width 0.2) (layer "B.Cu") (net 16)))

